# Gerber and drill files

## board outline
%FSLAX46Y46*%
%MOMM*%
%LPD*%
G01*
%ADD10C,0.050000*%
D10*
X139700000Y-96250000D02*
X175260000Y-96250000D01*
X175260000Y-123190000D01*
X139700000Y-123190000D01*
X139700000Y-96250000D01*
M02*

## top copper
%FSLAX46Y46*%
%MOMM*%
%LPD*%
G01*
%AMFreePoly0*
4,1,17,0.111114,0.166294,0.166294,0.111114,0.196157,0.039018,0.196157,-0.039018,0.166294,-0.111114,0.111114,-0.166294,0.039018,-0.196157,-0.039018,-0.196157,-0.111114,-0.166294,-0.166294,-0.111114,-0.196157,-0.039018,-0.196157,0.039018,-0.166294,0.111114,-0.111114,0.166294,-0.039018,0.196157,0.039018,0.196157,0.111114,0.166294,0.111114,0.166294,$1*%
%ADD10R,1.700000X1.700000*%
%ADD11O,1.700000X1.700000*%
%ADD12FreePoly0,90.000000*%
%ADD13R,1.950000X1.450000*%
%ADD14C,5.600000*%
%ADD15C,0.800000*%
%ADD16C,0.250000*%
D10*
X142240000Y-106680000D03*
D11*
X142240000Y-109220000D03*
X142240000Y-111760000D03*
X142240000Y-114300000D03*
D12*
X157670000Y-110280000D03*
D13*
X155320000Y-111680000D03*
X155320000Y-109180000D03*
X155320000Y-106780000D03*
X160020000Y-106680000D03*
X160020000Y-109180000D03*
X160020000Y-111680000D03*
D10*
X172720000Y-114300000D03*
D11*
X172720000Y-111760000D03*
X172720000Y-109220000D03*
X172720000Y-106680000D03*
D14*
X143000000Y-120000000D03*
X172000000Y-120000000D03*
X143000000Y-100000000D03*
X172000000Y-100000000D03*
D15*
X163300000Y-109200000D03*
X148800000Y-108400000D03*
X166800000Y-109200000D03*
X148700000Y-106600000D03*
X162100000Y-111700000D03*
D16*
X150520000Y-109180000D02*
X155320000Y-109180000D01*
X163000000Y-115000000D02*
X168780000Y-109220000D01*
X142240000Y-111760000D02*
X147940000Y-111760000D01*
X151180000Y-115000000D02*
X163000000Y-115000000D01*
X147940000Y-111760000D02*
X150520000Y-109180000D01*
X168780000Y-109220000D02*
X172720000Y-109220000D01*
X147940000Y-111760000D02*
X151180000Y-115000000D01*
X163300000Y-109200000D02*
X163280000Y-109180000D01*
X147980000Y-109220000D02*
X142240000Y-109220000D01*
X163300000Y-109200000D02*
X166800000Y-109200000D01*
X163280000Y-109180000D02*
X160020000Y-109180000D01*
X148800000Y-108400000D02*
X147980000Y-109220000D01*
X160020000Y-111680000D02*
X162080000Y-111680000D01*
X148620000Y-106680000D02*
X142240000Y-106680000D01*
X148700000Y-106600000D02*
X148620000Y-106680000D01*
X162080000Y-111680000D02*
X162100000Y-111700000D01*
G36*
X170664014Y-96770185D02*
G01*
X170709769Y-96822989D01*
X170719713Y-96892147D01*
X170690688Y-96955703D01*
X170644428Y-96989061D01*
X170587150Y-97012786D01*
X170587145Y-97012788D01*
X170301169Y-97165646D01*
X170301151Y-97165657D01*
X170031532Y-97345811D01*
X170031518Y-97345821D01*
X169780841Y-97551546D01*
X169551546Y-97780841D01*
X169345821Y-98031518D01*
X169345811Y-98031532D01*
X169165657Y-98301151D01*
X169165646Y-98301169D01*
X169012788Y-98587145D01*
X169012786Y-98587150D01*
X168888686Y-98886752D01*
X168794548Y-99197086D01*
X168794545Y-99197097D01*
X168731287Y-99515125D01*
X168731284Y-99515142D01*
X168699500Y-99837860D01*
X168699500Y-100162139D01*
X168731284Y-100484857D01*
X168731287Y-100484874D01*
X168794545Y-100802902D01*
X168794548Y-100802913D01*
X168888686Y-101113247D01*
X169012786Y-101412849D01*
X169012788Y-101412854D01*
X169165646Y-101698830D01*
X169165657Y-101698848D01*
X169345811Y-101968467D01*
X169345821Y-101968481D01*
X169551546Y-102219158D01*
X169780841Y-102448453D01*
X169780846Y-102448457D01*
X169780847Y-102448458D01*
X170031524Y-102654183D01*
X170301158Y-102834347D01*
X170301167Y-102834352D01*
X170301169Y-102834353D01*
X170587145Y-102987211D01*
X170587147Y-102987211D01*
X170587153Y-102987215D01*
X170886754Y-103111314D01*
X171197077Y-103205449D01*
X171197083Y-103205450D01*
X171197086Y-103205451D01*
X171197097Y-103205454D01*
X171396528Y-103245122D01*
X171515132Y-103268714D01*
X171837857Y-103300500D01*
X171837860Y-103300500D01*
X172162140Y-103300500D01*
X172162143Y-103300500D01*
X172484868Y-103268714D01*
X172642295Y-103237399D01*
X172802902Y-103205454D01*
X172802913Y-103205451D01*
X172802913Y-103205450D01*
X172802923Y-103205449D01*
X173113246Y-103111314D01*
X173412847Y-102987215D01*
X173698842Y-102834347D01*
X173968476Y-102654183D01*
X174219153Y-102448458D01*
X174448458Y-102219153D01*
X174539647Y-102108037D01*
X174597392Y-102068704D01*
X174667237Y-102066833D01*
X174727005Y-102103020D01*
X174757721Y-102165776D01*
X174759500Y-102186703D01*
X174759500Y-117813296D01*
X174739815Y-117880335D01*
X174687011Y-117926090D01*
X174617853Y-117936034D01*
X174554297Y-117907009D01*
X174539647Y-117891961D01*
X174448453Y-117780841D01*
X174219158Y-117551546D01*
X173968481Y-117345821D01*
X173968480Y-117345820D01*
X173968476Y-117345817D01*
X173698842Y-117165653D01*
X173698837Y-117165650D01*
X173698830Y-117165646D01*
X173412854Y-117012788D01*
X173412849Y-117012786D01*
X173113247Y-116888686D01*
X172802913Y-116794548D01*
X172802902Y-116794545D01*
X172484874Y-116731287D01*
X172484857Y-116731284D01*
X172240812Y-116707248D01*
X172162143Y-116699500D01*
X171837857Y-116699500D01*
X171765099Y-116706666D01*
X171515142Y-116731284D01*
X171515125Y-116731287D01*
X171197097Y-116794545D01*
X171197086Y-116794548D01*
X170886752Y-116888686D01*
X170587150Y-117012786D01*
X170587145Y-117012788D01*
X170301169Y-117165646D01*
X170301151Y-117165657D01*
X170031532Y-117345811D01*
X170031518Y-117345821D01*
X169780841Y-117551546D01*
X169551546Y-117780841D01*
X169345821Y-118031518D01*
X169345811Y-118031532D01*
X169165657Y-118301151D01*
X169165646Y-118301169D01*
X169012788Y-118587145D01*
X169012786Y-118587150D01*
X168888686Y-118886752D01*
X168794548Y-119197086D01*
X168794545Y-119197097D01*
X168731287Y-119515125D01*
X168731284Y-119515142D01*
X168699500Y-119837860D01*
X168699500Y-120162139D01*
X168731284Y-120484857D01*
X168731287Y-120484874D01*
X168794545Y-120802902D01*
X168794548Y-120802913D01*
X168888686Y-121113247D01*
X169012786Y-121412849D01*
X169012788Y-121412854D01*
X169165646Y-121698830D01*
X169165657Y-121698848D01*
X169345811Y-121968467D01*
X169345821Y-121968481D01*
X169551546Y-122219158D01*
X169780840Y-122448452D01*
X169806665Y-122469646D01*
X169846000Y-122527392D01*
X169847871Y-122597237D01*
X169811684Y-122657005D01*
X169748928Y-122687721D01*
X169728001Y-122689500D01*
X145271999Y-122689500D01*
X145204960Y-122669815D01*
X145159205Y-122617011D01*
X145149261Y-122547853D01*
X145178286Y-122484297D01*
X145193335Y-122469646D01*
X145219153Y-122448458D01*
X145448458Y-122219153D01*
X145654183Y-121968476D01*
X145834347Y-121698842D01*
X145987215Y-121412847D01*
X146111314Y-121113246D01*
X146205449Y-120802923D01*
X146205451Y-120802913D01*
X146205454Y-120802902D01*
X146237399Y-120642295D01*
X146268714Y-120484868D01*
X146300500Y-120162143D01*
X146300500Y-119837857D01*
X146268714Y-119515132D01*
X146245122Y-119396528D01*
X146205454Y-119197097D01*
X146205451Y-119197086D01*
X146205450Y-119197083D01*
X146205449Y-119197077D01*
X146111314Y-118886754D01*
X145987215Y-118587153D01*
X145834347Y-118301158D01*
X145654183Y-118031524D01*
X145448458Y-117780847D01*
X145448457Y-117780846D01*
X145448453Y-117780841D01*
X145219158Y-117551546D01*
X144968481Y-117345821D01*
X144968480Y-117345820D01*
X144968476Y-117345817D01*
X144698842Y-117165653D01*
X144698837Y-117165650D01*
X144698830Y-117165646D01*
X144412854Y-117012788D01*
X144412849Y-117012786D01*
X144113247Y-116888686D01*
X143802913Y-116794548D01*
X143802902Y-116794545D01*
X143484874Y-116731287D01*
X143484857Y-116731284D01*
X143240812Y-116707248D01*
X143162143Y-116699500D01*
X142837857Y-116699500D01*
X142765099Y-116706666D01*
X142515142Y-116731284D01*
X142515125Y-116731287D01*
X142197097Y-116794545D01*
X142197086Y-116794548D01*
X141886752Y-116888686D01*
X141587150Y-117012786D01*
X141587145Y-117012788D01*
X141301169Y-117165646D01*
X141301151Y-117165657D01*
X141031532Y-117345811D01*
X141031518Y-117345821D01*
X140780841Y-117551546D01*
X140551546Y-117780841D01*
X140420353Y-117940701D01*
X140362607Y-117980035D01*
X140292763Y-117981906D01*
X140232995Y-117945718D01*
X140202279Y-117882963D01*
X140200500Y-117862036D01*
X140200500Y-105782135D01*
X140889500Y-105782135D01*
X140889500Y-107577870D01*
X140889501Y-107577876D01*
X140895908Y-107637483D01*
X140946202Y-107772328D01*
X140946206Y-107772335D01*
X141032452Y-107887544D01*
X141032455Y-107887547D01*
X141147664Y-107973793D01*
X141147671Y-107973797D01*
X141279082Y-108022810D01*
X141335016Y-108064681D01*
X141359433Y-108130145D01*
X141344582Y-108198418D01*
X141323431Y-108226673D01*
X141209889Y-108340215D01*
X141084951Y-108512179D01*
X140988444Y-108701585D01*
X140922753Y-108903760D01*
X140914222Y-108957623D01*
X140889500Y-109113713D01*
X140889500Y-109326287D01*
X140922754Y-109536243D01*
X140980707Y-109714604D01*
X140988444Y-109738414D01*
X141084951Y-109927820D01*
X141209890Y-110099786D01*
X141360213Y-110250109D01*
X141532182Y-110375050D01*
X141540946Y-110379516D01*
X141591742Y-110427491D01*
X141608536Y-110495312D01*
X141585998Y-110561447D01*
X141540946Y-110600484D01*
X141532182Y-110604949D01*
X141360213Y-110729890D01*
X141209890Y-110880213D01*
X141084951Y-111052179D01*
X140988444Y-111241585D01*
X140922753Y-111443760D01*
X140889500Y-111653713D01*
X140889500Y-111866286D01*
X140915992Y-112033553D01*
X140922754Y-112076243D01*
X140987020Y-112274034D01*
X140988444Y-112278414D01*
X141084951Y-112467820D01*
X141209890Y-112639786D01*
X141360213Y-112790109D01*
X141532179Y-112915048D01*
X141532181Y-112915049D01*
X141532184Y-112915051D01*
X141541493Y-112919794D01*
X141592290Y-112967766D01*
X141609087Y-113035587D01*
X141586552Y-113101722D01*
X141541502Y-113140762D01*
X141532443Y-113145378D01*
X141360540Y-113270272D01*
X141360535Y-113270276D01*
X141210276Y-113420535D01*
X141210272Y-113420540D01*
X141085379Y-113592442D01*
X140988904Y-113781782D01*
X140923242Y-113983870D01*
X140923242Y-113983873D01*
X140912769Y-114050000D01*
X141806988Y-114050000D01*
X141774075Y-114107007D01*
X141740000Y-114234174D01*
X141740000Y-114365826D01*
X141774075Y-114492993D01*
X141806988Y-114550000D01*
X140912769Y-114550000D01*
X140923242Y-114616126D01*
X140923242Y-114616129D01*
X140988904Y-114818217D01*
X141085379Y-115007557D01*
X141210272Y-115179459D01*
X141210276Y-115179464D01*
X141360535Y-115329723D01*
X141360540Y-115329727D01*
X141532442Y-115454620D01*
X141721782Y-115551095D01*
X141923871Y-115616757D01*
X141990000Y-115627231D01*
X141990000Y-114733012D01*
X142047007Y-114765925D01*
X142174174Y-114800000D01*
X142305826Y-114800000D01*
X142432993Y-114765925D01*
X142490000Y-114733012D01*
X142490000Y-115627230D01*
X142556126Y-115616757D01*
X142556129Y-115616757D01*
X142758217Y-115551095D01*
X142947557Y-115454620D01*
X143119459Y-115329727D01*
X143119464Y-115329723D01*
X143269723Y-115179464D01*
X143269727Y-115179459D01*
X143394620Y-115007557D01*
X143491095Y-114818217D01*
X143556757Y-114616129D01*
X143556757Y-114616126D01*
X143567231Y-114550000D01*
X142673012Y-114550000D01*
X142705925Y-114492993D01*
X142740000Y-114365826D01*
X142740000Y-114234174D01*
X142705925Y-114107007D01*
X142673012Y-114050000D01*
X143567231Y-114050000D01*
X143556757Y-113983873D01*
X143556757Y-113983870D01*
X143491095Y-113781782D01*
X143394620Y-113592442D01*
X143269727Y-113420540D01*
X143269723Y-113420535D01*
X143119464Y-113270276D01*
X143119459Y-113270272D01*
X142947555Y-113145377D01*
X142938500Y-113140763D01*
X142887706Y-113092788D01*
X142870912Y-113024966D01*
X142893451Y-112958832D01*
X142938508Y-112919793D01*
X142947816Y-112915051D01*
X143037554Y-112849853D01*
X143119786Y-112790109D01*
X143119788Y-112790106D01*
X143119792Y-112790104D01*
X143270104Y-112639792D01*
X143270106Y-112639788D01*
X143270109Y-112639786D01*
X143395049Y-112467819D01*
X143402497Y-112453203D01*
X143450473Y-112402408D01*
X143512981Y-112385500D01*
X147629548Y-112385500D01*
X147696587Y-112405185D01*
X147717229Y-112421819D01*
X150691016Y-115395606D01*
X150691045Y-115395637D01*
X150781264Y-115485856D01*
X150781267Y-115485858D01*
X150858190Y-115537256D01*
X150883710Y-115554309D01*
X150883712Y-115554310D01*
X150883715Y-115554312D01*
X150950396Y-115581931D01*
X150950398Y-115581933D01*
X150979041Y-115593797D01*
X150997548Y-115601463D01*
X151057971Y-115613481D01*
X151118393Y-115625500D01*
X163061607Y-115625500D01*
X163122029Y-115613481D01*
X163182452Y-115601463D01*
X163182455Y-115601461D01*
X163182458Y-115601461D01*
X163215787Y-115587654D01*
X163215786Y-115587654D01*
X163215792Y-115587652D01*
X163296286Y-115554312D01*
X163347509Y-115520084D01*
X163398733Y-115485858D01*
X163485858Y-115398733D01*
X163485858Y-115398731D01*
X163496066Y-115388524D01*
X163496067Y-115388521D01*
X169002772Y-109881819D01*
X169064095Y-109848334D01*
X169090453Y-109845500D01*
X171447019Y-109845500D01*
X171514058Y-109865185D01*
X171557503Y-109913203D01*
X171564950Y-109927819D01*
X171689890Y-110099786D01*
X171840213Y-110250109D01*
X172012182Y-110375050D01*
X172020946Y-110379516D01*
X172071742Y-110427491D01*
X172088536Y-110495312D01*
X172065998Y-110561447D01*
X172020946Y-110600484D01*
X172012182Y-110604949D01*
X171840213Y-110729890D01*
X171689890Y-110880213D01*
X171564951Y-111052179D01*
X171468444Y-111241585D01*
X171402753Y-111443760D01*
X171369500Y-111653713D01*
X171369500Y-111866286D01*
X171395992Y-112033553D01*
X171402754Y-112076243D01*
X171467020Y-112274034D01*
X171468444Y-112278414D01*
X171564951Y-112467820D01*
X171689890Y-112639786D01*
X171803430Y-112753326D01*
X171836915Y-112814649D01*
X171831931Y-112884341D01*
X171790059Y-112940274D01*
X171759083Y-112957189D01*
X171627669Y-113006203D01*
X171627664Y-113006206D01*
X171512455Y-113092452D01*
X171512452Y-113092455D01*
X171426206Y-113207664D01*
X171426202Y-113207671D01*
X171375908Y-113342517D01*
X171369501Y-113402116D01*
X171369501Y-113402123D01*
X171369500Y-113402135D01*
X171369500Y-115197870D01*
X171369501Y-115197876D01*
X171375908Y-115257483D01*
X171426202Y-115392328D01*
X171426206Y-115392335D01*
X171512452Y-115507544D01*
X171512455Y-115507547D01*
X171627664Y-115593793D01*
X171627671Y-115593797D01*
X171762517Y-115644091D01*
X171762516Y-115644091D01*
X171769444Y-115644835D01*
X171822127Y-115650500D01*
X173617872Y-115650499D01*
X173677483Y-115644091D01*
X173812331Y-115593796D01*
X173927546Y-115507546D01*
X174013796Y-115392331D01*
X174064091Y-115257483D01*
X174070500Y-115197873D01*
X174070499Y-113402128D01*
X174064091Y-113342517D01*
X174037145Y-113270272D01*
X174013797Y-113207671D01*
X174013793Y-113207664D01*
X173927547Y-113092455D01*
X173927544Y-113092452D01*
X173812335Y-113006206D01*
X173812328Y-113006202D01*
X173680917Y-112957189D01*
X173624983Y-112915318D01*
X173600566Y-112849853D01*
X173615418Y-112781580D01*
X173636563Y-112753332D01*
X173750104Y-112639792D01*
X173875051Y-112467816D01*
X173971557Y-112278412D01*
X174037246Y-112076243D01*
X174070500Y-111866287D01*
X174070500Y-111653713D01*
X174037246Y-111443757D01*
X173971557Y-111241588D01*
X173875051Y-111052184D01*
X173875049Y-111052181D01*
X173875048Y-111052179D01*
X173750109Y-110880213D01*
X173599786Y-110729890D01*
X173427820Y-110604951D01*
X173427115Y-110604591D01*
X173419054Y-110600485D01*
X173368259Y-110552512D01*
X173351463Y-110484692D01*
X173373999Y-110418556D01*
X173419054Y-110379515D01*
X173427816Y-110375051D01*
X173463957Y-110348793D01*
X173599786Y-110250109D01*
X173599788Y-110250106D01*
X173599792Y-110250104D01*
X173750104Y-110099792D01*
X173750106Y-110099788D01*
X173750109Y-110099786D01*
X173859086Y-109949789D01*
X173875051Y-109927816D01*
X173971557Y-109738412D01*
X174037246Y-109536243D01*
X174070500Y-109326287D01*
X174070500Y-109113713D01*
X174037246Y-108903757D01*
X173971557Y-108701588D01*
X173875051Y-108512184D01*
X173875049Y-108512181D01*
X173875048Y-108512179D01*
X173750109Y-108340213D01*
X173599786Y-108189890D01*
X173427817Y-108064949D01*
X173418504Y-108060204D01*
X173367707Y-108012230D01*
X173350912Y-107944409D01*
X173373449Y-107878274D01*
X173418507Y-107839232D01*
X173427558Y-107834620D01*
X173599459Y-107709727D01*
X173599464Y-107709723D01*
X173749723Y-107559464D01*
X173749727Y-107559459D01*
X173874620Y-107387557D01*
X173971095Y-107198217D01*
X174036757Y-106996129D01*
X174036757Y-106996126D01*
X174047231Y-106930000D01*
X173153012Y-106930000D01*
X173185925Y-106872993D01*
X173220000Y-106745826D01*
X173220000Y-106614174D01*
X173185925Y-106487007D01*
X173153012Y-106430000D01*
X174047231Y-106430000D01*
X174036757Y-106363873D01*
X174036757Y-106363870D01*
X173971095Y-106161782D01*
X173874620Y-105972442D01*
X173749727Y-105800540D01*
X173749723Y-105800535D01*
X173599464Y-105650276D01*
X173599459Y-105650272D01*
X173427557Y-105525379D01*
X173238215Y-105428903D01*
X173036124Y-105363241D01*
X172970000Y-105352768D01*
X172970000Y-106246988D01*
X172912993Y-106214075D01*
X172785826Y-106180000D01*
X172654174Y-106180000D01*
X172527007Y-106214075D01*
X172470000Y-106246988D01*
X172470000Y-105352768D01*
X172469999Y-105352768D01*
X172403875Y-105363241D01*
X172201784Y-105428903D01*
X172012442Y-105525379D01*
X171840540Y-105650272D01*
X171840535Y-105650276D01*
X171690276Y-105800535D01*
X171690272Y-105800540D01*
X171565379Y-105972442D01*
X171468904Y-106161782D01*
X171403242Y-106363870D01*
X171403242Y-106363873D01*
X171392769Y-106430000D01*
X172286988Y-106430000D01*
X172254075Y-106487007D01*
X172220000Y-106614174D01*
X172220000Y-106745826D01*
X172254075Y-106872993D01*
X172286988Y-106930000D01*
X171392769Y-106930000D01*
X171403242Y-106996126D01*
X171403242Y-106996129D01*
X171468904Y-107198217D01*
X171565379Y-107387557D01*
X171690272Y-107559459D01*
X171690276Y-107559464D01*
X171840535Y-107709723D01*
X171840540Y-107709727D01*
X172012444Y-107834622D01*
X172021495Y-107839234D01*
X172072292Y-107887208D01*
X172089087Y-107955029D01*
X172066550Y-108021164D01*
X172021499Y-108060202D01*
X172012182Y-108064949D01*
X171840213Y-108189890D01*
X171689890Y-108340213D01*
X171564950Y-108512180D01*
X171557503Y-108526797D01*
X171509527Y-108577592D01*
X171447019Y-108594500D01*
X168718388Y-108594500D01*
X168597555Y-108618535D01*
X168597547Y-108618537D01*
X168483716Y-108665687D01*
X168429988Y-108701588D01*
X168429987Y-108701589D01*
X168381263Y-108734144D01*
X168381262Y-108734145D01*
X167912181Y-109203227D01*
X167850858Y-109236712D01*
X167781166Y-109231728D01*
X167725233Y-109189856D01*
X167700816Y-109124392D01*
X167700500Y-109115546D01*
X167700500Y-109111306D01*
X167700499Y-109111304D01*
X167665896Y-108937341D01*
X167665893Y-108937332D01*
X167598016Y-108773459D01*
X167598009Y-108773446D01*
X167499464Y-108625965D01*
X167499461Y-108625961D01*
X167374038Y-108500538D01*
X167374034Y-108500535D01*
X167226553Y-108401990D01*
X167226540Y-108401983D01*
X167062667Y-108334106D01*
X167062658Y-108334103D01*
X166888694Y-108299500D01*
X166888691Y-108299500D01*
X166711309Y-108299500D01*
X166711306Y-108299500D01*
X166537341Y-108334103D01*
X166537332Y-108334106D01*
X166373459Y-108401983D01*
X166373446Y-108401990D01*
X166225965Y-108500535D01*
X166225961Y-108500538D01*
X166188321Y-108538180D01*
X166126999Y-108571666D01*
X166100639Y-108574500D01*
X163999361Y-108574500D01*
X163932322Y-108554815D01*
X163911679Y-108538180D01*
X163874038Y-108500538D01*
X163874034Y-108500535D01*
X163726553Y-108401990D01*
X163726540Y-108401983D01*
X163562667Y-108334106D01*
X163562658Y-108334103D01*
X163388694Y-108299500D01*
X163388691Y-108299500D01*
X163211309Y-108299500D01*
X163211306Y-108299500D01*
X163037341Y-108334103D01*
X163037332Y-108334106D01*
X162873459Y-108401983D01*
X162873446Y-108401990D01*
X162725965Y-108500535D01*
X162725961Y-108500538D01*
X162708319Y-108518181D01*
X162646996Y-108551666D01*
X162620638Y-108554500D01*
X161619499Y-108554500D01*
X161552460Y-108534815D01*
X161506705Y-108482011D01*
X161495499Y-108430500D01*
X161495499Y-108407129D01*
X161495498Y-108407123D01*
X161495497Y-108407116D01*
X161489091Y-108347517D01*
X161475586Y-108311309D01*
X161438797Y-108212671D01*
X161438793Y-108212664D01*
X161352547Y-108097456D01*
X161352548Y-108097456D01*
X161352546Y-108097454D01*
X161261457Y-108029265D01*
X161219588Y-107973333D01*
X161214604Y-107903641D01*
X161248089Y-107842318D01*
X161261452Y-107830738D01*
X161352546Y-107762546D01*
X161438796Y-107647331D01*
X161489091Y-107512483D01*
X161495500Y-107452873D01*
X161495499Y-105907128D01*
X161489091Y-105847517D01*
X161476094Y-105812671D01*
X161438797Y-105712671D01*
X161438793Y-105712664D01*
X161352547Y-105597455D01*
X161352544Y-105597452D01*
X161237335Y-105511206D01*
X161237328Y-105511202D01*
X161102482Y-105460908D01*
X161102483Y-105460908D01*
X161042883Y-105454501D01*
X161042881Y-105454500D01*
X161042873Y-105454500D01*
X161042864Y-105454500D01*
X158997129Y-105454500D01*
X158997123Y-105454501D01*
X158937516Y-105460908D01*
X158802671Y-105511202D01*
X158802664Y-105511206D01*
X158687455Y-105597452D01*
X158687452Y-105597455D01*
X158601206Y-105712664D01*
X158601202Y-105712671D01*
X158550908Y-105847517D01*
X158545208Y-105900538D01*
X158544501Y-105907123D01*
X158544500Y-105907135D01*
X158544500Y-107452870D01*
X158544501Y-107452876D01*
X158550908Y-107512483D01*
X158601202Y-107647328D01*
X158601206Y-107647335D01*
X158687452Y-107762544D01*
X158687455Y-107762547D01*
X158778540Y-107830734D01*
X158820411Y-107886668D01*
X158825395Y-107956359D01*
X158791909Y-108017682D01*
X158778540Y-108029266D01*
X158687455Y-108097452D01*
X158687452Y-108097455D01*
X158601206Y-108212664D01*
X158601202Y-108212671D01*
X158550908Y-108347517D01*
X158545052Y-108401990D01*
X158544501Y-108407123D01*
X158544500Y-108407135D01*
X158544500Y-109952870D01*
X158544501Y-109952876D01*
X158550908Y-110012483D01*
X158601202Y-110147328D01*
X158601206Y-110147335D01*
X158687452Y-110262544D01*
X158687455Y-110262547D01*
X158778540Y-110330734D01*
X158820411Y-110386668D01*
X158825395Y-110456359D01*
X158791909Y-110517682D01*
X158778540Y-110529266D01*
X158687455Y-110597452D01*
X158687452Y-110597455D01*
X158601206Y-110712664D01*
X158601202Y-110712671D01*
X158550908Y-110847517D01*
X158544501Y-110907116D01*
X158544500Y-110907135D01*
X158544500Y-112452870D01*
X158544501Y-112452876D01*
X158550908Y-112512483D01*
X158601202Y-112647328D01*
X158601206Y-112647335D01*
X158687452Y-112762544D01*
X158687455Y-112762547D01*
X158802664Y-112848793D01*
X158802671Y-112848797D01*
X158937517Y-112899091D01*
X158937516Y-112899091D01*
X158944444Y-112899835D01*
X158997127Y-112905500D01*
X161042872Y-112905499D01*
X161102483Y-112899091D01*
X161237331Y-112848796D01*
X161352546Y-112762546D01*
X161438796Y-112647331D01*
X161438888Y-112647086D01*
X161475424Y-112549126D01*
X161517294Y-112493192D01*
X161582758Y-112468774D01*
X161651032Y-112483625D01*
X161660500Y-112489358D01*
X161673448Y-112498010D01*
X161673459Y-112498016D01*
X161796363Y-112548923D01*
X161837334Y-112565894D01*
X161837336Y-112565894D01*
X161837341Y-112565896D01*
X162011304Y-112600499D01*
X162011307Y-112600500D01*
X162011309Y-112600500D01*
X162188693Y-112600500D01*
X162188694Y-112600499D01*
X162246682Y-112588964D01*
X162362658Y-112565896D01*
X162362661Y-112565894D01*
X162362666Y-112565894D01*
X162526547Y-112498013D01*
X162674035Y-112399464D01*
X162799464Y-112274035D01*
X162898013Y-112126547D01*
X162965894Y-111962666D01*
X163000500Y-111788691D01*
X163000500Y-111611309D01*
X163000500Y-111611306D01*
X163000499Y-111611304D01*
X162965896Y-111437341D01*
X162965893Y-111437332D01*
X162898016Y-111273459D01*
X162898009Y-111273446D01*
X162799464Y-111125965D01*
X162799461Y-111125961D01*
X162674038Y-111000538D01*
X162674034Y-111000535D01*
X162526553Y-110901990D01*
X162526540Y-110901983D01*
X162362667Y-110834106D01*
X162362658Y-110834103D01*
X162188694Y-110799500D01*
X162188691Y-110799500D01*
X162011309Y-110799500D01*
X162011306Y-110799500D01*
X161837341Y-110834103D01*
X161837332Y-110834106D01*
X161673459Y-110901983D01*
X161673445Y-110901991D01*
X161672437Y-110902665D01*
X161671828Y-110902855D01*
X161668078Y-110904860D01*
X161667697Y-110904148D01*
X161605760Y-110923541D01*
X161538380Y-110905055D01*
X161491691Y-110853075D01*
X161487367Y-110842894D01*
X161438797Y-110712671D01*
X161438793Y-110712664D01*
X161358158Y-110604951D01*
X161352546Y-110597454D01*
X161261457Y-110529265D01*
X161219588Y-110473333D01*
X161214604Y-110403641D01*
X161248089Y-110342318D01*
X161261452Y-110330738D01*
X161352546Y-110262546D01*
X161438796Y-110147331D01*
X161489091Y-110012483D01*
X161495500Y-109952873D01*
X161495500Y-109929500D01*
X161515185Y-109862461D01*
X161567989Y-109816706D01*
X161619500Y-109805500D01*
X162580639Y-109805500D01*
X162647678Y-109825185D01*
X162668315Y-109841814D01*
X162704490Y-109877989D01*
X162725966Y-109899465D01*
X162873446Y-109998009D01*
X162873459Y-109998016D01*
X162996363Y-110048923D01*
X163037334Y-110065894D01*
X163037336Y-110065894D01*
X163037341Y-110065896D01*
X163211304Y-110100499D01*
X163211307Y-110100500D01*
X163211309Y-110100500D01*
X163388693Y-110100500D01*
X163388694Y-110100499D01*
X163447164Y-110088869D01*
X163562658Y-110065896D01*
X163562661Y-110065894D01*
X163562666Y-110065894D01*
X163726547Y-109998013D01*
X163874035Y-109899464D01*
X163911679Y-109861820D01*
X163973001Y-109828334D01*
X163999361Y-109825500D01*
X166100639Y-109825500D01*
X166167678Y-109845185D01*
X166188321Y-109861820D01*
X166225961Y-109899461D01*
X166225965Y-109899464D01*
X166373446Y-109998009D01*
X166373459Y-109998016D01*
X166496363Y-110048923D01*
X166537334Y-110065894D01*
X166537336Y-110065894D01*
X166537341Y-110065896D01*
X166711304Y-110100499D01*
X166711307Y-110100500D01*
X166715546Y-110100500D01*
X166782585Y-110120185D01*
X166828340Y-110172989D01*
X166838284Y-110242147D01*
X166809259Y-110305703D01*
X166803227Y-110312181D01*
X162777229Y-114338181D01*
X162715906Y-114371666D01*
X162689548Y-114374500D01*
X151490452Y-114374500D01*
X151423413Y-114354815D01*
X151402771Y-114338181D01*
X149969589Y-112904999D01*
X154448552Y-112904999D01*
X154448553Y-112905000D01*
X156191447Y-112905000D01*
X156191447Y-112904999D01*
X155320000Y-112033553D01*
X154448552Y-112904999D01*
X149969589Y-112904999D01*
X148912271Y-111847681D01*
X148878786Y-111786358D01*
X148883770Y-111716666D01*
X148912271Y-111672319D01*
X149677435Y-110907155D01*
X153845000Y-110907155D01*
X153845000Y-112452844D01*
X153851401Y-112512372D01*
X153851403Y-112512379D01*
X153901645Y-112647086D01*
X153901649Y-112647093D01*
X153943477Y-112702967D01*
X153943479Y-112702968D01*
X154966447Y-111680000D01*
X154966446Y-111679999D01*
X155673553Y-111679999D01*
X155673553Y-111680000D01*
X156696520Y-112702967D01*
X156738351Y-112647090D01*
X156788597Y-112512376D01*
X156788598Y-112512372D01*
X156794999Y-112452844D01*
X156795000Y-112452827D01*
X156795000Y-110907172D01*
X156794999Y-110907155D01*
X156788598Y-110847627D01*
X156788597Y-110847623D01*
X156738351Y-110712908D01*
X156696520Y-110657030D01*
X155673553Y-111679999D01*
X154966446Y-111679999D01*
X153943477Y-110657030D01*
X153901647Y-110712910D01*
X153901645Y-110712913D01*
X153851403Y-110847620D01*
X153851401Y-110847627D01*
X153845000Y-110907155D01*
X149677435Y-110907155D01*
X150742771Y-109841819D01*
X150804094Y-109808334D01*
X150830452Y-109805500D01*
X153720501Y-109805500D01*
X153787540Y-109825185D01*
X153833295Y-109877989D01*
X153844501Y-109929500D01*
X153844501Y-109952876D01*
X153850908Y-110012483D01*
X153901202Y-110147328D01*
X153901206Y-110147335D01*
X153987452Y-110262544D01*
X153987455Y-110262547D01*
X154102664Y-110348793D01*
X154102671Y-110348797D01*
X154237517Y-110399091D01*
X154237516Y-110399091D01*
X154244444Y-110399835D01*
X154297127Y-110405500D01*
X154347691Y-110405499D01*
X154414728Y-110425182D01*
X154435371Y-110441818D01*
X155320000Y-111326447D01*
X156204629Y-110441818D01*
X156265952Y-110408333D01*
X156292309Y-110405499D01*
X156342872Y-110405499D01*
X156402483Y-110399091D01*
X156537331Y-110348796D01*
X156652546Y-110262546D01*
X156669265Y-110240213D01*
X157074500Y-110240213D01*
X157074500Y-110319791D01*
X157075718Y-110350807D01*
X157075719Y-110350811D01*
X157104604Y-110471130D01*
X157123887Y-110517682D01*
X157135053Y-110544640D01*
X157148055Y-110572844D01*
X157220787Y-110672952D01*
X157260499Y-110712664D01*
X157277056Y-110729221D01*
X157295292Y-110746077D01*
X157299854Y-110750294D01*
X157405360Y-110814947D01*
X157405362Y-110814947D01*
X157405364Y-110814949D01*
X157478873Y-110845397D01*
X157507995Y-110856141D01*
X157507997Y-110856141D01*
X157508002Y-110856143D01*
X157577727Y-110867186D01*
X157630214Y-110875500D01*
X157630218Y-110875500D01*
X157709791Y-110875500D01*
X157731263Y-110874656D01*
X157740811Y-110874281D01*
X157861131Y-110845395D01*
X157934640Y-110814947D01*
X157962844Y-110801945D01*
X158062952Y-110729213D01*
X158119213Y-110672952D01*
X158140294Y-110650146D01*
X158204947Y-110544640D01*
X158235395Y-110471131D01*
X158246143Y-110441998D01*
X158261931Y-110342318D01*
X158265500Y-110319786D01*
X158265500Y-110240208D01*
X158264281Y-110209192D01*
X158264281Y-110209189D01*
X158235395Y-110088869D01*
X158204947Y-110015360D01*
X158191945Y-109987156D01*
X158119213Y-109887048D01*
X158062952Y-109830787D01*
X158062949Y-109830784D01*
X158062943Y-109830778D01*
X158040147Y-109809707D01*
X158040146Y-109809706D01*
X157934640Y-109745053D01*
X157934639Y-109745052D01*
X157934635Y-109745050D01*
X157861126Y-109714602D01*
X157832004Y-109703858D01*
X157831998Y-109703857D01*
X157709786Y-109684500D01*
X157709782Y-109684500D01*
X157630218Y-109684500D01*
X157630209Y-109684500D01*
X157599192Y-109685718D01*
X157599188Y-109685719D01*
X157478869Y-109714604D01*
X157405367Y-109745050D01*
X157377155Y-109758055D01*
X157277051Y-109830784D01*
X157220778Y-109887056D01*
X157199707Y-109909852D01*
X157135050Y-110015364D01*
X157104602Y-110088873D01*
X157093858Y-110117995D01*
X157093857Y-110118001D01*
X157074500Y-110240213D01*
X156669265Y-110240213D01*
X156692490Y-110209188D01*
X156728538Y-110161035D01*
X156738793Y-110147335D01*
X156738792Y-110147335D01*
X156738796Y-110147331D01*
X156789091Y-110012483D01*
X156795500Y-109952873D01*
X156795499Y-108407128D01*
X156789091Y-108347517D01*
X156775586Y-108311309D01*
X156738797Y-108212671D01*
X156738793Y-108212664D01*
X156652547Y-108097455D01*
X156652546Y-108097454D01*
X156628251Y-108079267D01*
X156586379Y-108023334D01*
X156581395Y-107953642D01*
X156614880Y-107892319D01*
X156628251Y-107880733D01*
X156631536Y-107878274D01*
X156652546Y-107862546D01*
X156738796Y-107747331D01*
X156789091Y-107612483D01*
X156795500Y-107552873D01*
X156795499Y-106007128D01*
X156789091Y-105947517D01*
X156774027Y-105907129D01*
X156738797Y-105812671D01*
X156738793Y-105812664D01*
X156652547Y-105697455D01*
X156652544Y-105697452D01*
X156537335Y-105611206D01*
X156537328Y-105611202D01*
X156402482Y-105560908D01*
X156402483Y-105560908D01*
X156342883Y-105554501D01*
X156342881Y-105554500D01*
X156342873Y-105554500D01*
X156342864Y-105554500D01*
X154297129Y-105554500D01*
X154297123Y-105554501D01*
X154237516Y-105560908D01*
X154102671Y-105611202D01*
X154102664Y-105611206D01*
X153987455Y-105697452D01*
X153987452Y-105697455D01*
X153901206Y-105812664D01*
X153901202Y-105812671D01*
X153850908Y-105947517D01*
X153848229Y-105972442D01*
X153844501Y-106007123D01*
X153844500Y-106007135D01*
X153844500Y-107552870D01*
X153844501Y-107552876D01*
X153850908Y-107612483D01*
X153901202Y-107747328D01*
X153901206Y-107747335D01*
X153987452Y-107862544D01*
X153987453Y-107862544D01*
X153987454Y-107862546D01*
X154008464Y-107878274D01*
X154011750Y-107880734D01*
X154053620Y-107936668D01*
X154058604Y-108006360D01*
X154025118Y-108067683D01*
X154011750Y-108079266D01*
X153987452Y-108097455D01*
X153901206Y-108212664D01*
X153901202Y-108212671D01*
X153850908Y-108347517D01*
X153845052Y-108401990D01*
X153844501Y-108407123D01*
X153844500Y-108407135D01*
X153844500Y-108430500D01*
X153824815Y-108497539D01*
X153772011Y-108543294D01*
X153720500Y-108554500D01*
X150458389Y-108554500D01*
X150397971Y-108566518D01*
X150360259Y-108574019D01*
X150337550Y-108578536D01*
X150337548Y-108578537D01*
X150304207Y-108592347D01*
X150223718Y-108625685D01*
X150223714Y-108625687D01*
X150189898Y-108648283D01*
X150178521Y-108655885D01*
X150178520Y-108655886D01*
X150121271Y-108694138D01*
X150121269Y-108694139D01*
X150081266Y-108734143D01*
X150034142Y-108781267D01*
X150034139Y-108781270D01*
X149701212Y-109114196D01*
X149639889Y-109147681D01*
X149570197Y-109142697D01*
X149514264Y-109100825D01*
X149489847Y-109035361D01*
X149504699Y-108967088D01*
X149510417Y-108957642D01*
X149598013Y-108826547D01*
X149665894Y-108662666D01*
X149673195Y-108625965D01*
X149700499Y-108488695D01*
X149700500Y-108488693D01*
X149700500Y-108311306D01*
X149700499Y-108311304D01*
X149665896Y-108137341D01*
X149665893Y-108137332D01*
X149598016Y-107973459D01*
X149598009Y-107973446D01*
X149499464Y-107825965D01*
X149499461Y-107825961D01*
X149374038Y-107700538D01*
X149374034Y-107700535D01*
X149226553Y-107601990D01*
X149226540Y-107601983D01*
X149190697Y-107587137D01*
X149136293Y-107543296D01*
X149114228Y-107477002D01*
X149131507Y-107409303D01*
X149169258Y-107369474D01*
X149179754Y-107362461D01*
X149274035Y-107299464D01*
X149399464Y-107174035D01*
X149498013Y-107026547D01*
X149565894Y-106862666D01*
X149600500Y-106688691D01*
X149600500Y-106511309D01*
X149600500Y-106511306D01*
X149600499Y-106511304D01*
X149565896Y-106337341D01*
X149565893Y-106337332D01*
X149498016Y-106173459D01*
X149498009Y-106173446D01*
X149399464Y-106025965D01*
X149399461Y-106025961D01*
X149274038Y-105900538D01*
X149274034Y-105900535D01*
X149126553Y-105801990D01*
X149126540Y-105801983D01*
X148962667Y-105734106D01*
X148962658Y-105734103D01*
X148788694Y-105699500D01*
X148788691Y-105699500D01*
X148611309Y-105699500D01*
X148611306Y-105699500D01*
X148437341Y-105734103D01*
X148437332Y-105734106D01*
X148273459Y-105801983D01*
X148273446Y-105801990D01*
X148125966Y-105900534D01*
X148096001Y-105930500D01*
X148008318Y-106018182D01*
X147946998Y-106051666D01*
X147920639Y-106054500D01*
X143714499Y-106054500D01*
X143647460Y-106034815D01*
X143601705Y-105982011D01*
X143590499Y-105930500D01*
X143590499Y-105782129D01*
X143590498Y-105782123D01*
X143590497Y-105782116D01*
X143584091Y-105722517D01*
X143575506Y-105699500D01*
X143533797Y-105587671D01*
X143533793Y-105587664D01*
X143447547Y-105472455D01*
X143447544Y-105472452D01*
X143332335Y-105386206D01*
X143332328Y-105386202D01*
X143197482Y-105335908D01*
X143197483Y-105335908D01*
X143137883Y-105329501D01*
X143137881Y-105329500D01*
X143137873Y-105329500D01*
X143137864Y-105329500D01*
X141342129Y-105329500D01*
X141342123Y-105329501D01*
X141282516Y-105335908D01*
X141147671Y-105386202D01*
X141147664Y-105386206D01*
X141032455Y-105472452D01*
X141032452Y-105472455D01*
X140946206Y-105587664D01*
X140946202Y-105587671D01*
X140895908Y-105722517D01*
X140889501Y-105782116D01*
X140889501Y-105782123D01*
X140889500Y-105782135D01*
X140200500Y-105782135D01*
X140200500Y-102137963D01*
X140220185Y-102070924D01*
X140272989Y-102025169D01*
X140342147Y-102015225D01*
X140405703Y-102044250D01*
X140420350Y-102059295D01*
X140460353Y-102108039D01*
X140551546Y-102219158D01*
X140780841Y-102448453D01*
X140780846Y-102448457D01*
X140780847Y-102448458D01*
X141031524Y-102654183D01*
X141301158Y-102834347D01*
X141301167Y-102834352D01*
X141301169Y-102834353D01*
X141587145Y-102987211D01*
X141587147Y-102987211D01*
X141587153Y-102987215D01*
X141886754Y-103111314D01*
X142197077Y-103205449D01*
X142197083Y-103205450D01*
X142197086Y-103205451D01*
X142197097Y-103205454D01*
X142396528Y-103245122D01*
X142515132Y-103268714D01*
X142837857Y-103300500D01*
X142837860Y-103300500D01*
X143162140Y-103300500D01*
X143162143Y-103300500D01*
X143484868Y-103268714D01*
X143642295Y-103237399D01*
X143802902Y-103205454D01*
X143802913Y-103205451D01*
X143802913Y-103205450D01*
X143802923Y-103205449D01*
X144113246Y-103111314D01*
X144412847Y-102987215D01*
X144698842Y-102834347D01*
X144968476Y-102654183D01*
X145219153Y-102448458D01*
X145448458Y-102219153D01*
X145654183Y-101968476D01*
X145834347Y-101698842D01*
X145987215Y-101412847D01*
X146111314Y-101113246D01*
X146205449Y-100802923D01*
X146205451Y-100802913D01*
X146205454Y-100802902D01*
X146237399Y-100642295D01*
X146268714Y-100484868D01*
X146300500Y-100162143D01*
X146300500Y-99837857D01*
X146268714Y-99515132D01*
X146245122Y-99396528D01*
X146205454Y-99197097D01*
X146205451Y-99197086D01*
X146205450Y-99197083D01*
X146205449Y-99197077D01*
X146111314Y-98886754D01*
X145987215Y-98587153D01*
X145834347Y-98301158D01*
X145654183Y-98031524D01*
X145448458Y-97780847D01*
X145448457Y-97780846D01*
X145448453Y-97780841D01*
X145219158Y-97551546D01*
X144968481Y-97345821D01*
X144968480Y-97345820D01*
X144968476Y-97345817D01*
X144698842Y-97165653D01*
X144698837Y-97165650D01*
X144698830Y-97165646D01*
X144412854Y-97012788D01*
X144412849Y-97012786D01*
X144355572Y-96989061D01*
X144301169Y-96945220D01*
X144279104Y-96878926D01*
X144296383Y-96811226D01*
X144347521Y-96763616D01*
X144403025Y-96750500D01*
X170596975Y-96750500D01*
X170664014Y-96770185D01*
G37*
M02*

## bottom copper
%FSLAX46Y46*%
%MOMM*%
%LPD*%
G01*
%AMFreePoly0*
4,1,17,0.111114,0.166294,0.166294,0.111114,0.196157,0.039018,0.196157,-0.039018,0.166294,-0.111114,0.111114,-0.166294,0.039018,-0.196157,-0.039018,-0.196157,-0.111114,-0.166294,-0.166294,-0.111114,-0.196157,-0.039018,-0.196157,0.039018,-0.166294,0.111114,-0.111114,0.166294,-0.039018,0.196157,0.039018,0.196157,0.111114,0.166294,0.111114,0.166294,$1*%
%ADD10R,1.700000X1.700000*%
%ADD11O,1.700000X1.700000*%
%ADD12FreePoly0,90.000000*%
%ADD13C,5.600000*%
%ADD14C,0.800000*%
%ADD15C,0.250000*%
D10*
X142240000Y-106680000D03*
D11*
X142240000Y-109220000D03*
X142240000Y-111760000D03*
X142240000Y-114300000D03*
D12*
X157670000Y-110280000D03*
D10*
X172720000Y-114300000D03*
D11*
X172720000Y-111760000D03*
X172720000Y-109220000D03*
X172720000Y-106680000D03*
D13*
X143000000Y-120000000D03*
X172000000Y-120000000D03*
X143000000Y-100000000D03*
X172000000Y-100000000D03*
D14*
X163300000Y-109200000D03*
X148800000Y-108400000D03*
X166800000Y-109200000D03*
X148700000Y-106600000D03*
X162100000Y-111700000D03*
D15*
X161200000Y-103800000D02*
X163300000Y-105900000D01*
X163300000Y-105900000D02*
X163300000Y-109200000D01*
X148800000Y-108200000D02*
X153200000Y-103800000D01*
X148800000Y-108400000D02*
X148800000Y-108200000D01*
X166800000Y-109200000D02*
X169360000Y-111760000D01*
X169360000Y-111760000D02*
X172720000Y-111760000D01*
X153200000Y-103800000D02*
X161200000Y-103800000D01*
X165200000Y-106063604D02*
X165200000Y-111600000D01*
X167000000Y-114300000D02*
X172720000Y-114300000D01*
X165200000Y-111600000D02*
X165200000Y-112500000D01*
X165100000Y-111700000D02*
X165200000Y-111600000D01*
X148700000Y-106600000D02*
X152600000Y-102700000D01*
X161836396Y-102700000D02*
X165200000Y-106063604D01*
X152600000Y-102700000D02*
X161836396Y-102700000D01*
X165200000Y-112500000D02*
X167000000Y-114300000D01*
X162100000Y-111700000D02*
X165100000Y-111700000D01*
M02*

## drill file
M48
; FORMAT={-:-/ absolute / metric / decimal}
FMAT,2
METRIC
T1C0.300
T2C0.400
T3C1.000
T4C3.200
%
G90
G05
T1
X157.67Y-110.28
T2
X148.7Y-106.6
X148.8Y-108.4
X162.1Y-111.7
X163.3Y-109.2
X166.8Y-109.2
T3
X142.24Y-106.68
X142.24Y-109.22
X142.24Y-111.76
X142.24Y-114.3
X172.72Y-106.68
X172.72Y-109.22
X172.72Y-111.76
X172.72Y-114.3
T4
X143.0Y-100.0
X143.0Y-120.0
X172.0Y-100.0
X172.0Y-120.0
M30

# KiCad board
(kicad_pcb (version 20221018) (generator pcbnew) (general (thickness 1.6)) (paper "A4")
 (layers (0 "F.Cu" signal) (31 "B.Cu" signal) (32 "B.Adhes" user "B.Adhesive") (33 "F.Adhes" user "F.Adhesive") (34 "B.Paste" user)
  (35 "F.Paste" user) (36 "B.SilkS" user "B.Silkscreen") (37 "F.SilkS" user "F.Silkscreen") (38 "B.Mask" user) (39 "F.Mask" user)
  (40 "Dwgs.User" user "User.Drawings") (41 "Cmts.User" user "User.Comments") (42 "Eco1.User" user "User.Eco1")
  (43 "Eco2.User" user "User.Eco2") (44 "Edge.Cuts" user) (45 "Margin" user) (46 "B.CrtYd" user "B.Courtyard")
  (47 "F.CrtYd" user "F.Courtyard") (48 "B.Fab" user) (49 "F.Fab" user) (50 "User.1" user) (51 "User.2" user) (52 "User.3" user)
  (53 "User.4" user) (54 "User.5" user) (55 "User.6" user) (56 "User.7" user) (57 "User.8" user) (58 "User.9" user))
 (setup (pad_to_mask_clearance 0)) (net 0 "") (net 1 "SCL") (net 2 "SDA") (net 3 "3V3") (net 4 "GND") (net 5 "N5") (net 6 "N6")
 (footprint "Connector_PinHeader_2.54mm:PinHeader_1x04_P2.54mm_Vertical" (layer "F.Cu") (at 142.24 106.68)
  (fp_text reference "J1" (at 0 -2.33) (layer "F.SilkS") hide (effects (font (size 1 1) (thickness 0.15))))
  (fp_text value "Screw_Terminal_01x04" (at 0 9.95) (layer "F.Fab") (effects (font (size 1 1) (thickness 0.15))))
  (pad "1" thru_hole rect (at 0 0) (size 1.7 1.7) (drill 1) (layers "*.Cu" "*.Mask") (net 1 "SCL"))
  (pad "2" thru_hole oval (at 0 2.54) (size 1.7 1.7) (drill 1) (layers "*.Cu" "*.Mask") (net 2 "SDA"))
  (pad "3" thru_hole oval (at 0 5.08) (size 1.7 1.7) (drill 1) (layers "*.Cu" "*.Mask") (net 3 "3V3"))
  (pad "4" thru_hole oval (at 0 7.62) (size 1.7 1.7) (drill 1) (layers "*.Cu" "*.Mask") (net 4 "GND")))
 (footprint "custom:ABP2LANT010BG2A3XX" (layer "F.Cu") (at 154.07 113.28 90)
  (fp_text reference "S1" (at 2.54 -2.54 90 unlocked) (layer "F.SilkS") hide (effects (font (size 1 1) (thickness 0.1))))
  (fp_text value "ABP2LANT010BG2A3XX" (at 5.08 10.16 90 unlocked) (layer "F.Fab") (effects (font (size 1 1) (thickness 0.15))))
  (pad "" thru_hole custom (at 3 3.6 90) (size 0.4 0.4) (drill 0.3) (layers "*.Cu" "*.Mask") (solder_mask_margin 0.6) (clearance 0.39)
   (thermal_bridge_angle 90) (options (clearance outline) (anchor circle)) (primitives))
  (pad "1" smd rect (at 1.6 1.25 90) (size 1.45 1.95) (layers "F.Cu" "F.Paste" "F.Mask") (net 4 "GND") (thermal_bridge_angle 45))
  (pad "2" smd rect (at 4.1 1.25 90) (size 1.45 1.95) (layers "F.Cu" "F.Paste" "F.Mask") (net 3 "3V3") (thermal_bridge_angle 45))
  (pad "3" smd rect (at 6.5 1.25 90) (size 1.45 1.95) (layers "F.Cu" "F.Paste" "F.Mask") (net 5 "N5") (thermal_bridge_angle 45))
  (pad "4" smd rect (at 6.6 5.95 90) (size 1.45 1.95) (layers "F.Cu" "F.Paste" "F.Mask") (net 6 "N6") (thermal_bridge_angle 45))
  (pad "5" smd rect (at 4.1 5.95 90) (size 1.45 1.95) (layers "F.Cu" "F.Paste" "F.Mask") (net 2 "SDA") (thermal_bridge_angle 45))
  (pad "6" smd rect (at 1.6 5.95 90) (size 1.45 1.95) (layers "F.Cu" "F.Paste" "F.Mask") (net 1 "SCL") (thermal_bridge_angle 45)))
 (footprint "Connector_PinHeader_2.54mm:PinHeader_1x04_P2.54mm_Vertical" (layer "F.Cu") (at 172.72 114.3 180)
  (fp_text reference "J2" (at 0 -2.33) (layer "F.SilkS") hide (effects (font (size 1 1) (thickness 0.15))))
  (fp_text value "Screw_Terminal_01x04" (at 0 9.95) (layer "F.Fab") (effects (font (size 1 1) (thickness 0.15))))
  (pad "1" thru_hole rect (at 0 0 180) (size 1.7 1.7) (drill 1) (layers "*.Cu" "*.Mask") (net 1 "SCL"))
  (pad "2" thru_hole oval (at 0 2.54 180) (size 1.7 1.7) (drill 1) (layers "*.Cu" "*.Mask") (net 2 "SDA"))
  (pad "3" thru_hole oval (at 0 5.08 180) (size 1.7 1.7) (drill 1) (layers "*.Cu" "*.Mask") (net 3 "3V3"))
  (pad "4" thru_hole oval (at 0 7.62 180) (size 1.7 1.7) (drill 1) (layers "*.Cu" "*.Mask") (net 4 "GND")))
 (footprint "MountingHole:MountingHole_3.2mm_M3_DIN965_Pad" (layer "F.Cu") (at 143 120)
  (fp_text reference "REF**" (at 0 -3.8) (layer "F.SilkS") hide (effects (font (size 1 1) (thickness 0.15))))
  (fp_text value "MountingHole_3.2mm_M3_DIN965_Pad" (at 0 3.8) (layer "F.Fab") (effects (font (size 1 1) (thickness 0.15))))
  (pad "1" thru_hole circle (at 0 0) (size 5.6 5.6) (drill 3.2) (layers "*.Cu" "*.Mask")))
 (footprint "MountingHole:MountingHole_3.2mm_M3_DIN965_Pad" (layer "F.Cu") (at 172 120)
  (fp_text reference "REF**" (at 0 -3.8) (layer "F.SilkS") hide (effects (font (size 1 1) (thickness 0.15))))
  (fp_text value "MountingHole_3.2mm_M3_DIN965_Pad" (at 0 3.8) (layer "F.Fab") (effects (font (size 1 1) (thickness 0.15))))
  (pad "1" thru_hole circle (at 0 0) (size 5.6 5.6) (drill 3.2) (layers "*.Cu" "*.Mask")))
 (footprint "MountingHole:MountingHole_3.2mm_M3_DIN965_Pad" (layer "F.Cu") (at 143 100)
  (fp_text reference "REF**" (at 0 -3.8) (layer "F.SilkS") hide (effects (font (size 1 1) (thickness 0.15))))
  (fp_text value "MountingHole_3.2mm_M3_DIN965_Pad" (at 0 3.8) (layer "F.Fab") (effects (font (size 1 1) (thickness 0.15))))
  (pad "1" thru_hole circle (at 0 0) (size 5.6 5.6) (drill 3.2) (layers "*.Cu" "*.Mask")))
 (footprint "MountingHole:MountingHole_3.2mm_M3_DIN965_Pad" (layer "F.Cu") (at 172 100)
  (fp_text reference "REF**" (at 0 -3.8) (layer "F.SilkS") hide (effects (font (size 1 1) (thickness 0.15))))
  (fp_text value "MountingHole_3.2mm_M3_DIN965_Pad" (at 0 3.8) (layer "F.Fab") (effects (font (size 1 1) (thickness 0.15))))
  (pad "1" thru_hole circle (at 0 0) (size 5.6 5.6) (drill 3.2) (layers "*.Cu" "*.Mask")))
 (gr_rect (start 139.7 96.25) (end 175.26 123.19) (stroke (width 0.05) (type default)) (fill none) (layer "Edge.Cuts"))
 (segment (start 150.52 109.18) (end 155.32 109.18) (width 0.25) (layer "F.Cu") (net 3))
 (segment (start 163 115) (end 168.78 109.22) (width 0.25) (layer "F.Cu") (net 3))
 (segment (start 142.24 111.76) (end 147.94 111.76) (width 0.25) (layer "F.Cu") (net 3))
 (segment (start 151.18 115) (end 163 115) (width 0.25) (layer "F.Cu") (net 3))
 (segment (start 147.94 111.76) (end 150.52 109.18) (width 0.25) (layer "F.Cu") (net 3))
 (segment (start 168.78 109.22) (end 172.72 109.22) (width 0.25) (layer "F.Cu") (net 3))
 (segment (start 147.94 111.76) (end 151.18 115) (width 0.25) (layer "F.Cu") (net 3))
 (segment (start 163.3 109.2) (end 163.28 109.18) (width 0.25) (layer "F.Cu") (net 2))
 (segment (start 147.98 109.22) (end 142.24 109.22) (width 0.25) (layer "F.Cu") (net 2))
 (segment (start 163.3 109.2) (end 166.8 109.2) (width 0.25) (layer "F.Cu") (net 2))
 (segment (start 163.28 109.18) (end 160.02 109.18) (width 0.25) (layer "F.Cu") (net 2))
 (segment (start 148.8 108.4) (end 147.98 109.22) (width 0.25) (layer "F.Cu") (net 2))
 (via (at 163.3 109.2) (size 0.8) (drill 0.4) (layers "F.Cu" "B.Cu") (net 2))
 (via (at 148.8 108.4) (size 0.8) (drill 0.4) (layers "F.Cu" "B.Cu") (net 2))
 (via (at 166.8 109.2) (size 0.8) (drill 0.4) (layers "F.Cu" "B.Cu") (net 2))
 (segment (start 161.2 103.8) (end 163.3 105.9) (width 0.25) (layer "B.Cu") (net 2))
 (segment (start 163.3 105.9) (end 163.3 109.2) (width 0.25) (layer "B.Cu") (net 2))
 (segment (start 148.8 108.2) (end 153.2 103.8) (width 0.25) (layer "B.Cu") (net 2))
 (segment (start 148.8 108.4) (end 148.8 108.2) (width 0.25) (layer "B.Cu") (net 2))
 (segment (start 166.8 109.2) (end 169.36 111.76) (width 0.25) (layer "B.Cu") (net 2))
 (segment (start 169.36 111.76) (end 172.72 111.76) (width 0.25) (layer "B.Cu") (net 2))
 (segment (start 153.2 103.8) (end 161.2 103.8) (width 0.25) (layer "B.Cu") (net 2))
 (segment (start 160.02 111.68) (end 162.08 111.68) (width 0.25) (layer "F.Cu") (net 1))
 (segment (start 148.62 106.68) (end 142.24 106.68) (width 0.25) (layer "F.Cu") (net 1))
 (segment (start 148.7 106.6) (end 148.62 106.68) (width 0.25) (layer "F.Cu") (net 1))
 (segment (start 162.08 111.68) (end 162.1 111.7) (width 0.25) (layer "F.Cu") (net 1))
 (via (at 148.7 106.6) (size 0.8) (drill 0.4) (layers "F.Cu" "B.Cu") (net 1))
 (via (at 162.1 111.7) (size 0.8) (drill 0.4) (layers "F.Cu" "B.Cu") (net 1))
 (segment (start 165.2 106.063604) (end 165.2 111.6) (width 0.25) (layer "B.Cu") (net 1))
 (segment (start 167 114.3) (end 172.72 114.3) (width 0.25) (layer "B.Cu") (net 1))
 (segment (start 165.2 111.6) (end 165.2 112.5) (width 0.25) (layer "B.Cu") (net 1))
 (segment (start 165.1 111.7) (end 165.2 111.6) (width 0.25) (layer "B.Cu") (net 1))
 (segment (start 148.7 106.6) (end 152.6 102.7) (width 0.25) (layer "B.Cu") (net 1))
 (segment (start 161.836396 102.7) (end 165.2 106.063604) (width 0.25) (layer "B.Cu") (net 1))
 (segment (start 152.6 102.7) (end 161.836396 102.7) (width 0.25) (layer "B.Cu") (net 1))
 (segment (start 165.2 112.5) (end 167 114.3) (width 0.25) (layer "B.Cu") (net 1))
 (segment (start 162.1 111.7) (end 165.1 111.7) (width 0.25) (layer "B.Cu") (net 1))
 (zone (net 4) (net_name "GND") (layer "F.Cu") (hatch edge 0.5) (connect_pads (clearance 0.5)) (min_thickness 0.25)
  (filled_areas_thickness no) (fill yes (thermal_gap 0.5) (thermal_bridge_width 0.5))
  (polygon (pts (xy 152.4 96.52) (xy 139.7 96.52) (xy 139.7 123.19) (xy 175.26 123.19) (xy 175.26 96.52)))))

